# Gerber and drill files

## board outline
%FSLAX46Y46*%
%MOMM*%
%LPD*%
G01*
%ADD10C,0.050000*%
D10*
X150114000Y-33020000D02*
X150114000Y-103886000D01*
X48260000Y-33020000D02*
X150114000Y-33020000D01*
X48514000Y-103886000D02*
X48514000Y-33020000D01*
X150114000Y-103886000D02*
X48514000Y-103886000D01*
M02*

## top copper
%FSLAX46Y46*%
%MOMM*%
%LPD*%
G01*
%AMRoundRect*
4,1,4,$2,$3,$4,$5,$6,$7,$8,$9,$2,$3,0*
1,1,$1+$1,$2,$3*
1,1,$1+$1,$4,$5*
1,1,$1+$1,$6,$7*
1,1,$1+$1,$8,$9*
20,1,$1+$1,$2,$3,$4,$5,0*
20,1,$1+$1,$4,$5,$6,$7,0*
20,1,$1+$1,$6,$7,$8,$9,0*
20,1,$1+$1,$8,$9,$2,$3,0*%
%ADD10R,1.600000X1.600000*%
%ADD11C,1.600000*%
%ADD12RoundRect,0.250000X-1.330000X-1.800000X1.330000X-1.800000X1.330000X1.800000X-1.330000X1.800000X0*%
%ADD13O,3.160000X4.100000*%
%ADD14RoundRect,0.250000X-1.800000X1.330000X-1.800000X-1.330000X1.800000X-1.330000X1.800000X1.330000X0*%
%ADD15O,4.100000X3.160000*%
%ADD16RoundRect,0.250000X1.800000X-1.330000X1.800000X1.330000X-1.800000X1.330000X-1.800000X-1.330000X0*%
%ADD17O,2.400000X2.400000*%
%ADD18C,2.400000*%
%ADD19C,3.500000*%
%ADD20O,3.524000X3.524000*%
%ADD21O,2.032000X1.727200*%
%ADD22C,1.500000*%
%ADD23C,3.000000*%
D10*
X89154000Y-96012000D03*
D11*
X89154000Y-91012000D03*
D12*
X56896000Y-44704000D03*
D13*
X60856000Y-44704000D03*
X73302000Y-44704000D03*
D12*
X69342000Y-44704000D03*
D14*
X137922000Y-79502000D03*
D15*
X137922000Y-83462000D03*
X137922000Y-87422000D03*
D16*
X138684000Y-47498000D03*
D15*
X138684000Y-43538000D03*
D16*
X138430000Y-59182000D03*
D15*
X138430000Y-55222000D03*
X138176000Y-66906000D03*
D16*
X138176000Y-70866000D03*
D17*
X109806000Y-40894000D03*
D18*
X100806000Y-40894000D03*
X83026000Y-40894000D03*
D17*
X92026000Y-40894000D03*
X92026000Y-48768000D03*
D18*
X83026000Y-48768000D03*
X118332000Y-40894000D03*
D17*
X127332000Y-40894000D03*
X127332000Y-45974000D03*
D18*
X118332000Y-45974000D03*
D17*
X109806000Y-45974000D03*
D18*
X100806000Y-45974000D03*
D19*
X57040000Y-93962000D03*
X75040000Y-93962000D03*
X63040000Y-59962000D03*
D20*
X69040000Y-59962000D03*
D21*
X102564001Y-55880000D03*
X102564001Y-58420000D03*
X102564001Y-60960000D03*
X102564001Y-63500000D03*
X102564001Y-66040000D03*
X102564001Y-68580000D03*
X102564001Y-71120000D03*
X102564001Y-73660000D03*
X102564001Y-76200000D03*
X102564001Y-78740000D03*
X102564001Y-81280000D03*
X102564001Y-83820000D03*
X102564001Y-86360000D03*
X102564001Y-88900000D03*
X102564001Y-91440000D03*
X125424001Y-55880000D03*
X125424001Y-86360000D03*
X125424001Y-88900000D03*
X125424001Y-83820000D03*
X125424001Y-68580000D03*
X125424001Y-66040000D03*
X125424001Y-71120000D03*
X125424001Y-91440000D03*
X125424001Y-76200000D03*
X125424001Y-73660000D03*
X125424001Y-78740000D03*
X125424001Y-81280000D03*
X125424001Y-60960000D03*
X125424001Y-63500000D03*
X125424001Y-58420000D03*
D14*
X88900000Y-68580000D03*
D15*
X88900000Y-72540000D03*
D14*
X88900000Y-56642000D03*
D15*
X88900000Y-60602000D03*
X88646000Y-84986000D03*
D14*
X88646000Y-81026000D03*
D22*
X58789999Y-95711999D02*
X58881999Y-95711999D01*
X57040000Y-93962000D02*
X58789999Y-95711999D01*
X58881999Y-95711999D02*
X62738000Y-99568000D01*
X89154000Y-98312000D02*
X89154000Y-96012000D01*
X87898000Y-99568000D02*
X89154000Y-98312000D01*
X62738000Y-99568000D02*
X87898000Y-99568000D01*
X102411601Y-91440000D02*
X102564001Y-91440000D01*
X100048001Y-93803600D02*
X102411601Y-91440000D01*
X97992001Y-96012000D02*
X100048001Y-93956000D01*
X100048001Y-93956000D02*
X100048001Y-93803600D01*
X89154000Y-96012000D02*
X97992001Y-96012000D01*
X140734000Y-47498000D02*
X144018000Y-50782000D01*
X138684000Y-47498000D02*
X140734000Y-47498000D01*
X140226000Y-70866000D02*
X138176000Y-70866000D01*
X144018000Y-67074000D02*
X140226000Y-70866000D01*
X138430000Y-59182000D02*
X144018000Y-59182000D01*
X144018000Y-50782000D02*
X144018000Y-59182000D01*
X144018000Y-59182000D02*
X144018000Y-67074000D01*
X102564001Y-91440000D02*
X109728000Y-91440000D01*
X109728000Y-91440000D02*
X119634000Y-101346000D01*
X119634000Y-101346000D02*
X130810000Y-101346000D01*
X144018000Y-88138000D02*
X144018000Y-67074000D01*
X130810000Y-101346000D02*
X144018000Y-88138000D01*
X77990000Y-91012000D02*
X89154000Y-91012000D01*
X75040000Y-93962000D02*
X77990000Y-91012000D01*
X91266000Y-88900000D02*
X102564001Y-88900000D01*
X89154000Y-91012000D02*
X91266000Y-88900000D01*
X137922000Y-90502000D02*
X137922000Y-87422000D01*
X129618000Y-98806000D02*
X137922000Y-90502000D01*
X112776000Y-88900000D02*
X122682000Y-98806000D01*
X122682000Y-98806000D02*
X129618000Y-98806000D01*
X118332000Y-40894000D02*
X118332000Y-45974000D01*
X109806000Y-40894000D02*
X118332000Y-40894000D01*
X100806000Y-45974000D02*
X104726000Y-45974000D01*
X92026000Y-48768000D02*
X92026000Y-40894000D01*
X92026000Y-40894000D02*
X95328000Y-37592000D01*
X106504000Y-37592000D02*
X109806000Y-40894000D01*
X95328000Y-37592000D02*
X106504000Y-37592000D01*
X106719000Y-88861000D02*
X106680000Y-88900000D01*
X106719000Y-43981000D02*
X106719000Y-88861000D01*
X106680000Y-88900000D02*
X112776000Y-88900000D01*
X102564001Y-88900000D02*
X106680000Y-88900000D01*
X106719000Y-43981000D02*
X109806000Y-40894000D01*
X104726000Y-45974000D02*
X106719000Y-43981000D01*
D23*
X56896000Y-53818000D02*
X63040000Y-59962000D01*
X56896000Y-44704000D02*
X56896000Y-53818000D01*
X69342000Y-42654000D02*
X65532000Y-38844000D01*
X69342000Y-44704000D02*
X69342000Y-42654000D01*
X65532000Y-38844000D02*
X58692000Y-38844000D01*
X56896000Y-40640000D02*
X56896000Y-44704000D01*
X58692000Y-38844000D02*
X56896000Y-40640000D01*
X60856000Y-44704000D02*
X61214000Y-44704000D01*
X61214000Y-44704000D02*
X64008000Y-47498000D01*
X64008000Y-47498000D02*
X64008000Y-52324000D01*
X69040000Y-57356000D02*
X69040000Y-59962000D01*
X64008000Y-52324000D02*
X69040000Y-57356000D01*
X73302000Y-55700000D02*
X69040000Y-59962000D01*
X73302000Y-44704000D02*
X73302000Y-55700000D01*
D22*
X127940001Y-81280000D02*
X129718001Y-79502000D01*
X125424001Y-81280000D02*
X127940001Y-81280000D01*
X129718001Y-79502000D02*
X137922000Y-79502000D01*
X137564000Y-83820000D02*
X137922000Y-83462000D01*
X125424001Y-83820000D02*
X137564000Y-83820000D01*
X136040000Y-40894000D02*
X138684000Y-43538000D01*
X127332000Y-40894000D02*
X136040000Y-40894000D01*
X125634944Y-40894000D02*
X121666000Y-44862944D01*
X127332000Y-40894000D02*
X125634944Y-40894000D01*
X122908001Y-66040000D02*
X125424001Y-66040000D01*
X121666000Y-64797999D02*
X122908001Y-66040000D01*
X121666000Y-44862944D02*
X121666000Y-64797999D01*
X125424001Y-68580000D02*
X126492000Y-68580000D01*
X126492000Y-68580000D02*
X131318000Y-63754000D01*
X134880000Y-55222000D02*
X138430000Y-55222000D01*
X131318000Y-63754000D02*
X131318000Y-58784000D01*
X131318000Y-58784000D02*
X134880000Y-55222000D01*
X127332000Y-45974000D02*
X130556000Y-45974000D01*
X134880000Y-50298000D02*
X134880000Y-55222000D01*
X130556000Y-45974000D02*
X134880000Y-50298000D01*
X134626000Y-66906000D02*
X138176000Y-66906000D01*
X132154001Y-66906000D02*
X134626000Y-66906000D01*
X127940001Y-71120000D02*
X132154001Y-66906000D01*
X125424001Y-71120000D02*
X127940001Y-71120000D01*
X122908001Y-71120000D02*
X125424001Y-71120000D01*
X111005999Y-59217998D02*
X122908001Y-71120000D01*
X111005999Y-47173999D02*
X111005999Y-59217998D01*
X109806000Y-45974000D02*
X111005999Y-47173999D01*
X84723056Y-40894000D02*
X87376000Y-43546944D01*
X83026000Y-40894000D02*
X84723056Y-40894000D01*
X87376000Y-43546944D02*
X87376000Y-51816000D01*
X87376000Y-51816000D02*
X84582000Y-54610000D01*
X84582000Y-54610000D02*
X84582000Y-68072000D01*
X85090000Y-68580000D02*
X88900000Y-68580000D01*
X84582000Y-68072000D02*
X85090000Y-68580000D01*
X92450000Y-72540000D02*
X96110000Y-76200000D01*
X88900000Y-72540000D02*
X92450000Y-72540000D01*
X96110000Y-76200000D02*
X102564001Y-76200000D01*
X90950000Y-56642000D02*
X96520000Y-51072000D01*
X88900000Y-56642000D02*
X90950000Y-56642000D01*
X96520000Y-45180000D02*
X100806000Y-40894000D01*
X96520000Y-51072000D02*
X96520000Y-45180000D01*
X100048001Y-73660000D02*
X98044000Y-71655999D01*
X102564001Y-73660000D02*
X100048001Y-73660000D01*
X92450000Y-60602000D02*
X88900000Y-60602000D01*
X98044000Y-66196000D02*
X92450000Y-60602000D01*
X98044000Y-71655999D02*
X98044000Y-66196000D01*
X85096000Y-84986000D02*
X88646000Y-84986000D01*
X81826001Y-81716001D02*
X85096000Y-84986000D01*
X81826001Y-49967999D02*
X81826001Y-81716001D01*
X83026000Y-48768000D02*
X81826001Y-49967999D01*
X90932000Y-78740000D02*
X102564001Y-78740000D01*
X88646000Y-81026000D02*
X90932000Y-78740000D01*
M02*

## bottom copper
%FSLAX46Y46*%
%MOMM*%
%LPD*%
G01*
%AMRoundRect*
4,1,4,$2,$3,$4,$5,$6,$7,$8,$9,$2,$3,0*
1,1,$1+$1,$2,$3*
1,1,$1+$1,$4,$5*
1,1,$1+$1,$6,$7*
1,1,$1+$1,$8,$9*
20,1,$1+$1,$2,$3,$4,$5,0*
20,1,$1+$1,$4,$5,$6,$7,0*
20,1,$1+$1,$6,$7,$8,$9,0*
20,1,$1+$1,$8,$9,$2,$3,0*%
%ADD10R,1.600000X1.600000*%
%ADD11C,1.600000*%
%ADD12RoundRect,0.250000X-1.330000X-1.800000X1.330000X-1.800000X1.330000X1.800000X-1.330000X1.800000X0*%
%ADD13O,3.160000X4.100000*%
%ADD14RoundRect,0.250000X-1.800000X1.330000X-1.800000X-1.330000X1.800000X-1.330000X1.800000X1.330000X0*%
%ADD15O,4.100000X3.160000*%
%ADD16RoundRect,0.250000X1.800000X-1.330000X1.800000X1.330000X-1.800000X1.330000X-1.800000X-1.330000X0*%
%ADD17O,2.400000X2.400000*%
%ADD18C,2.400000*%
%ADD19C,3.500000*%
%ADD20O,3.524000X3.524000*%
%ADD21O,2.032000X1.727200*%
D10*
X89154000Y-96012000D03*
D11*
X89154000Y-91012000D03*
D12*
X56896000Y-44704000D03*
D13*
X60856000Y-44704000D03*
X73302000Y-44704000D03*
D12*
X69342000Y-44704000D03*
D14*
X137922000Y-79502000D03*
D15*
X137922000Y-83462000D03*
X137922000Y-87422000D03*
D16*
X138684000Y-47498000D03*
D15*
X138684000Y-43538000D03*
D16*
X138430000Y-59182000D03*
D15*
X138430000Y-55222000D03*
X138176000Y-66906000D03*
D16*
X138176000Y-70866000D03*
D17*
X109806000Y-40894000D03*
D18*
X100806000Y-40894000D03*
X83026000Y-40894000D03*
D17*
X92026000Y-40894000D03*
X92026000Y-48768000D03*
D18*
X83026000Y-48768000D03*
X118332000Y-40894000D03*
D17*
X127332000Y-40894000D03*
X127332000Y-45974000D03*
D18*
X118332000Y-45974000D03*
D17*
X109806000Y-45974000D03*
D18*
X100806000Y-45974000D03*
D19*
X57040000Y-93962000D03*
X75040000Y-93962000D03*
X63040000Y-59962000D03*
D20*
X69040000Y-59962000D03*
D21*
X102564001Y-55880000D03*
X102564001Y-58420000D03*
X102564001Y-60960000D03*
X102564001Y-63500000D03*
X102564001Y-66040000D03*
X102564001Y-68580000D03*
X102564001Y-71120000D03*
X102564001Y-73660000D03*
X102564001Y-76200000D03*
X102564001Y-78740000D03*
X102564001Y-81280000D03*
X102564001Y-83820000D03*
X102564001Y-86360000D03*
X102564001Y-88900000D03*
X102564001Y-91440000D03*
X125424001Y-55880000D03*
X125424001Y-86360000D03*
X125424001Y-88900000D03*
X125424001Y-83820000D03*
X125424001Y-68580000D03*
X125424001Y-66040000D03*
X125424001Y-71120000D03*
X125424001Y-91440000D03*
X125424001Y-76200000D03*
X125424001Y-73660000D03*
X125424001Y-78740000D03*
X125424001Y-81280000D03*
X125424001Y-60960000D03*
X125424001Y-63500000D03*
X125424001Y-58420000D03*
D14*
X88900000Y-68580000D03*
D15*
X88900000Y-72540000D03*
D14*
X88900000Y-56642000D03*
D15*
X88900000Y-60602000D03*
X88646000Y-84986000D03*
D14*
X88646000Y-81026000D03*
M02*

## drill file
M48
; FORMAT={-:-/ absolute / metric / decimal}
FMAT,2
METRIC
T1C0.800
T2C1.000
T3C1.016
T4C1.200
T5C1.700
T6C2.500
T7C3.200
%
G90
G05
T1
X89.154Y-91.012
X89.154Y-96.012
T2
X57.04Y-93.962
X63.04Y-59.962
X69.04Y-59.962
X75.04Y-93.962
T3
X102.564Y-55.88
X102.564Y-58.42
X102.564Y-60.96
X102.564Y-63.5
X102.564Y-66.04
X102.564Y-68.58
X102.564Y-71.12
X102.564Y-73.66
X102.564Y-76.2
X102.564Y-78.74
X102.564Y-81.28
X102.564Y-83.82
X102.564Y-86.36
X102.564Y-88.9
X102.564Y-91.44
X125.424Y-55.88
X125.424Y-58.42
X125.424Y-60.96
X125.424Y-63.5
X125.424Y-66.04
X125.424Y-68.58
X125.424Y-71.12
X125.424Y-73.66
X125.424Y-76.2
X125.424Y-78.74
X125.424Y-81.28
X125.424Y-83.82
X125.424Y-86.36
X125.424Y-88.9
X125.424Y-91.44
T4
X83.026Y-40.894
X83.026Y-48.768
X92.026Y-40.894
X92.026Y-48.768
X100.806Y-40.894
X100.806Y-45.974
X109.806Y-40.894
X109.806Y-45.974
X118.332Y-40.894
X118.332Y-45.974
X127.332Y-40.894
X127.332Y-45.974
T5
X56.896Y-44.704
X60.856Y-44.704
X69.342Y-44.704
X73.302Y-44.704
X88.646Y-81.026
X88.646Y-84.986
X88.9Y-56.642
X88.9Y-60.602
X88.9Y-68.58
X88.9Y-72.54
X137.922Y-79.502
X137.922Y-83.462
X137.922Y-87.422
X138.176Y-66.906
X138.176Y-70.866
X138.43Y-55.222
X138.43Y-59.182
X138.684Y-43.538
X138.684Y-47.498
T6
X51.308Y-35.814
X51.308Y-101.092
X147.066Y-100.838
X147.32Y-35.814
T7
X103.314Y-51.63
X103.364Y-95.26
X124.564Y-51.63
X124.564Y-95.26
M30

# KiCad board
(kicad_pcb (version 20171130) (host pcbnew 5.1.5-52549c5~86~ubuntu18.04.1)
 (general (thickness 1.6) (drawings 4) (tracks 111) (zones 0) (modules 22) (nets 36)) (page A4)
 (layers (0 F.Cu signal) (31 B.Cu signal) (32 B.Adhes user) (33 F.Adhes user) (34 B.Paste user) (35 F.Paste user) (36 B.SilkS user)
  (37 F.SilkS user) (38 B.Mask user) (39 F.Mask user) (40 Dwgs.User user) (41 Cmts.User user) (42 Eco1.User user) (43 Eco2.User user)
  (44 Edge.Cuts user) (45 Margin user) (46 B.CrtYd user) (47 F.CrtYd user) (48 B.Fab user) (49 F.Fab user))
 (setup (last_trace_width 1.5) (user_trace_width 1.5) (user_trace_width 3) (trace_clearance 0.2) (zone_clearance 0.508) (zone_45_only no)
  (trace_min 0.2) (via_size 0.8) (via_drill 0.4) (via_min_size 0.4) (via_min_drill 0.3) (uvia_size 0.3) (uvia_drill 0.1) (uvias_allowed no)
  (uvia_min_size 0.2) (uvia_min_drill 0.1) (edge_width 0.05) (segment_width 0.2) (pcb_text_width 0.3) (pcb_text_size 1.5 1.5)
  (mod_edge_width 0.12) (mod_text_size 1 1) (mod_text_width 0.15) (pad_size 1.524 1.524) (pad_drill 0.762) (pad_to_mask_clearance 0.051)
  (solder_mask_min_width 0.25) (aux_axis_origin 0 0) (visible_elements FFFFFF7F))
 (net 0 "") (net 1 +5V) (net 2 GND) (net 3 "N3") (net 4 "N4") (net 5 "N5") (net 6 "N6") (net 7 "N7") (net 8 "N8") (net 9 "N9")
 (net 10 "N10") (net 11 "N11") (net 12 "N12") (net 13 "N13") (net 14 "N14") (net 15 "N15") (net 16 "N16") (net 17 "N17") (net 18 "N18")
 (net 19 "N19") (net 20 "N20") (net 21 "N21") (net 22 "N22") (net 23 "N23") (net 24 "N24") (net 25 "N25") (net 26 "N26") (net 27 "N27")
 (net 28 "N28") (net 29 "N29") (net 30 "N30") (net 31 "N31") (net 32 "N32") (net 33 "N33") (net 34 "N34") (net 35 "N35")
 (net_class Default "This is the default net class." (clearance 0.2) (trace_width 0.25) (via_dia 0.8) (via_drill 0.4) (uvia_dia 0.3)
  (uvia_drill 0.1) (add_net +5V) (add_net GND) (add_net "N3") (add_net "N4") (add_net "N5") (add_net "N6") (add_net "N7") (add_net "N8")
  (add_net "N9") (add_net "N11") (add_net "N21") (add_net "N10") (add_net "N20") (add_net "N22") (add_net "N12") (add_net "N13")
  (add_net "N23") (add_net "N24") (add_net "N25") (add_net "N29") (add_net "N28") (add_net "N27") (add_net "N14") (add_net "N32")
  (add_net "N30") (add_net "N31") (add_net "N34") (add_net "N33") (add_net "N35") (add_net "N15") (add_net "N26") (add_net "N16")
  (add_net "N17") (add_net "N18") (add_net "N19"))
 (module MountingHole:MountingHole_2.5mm (layer F.Cu) (at 51.308 35.814)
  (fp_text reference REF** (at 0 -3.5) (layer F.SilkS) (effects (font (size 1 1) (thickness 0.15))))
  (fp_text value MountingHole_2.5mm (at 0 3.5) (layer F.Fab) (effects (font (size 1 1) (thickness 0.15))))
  (pad 1 np_thru_hole circle (at 0 0) (size 2.5 2.5) (drill 2.5) (layers *.Cu *.Mask)))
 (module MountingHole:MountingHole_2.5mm (layer F.Cu) (at 51.308 101.092)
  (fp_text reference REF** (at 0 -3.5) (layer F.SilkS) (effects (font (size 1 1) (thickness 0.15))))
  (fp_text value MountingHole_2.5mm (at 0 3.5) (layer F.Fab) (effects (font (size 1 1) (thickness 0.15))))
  (pad 1 np_thru_hole circle (at 0 0) (size 2.5 2.5) (drill 2.5) (layers *.Cu *.Mask)))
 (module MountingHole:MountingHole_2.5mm (layer F.Cu) (at 147.066 100.838)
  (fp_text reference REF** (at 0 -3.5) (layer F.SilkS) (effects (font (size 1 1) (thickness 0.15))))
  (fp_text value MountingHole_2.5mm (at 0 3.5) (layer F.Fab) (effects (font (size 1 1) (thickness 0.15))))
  (pad 1 np_thru_hole circle (at 0 0) (size 2.5 2.5) (drill 2.5) (layers *.Cu *.Mask)))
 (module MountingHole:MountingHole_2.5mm (layer F.Cu) (at 147.32 35.814)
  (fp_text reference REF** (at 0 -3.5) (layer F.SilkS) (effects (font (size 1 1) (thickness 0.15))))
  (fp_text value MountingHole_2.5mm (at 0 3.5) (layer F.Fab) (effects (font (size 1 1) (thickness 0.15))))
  (pad 1 np_thru_hole circle (at 0 0) (size 2.5 2.5) (drill 2.5) (layers *.Cu *.Mask)))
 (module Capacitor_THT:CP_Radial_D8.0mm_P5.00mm (layer F.Cu) (at 89.154 96.012 90)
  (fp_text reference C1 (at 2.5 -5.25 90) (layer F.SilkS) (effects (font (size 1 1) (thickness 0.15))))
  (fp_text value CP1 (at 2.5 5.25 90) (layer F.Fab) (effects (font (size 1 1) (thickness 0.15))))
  (pad 1 thru_hole rect (at 0 0 90) (size 1.6 1.6) (drill 0.8) (layers *.Cu *.Mask) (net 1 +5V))
  (pad 2 thru_hole circle (at 5 0 90) (size 1.6 1.6) (drill 0.8) (layers *.Cu *.Mask) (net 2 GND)))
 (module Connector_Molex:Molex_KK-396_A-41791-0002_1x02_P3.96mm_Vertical (layer F.Cu) (at 56.896 44.704)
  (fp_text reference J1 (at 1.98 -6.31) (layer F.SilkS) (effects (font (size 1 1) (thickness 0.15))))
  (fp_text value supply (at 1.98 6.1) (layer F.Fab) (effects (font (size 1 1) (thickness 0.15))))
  (pad 1 thru_hole roundrect (at 0 0) (size 3.16 4.1) (drill 1.7) (layers *.Cu *.Mask) (roundrect_rratio 0.079114) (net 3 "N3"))
  (pad 2 thru_hole oval (at 3.96 0) (size 3.16 4.1) (drill 1.7) (layers *.Cu *.Mask) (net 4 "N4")))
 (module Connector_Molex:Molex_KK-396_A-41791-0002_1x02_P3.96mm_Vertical (layer F.Cu) (at 69.342 44.704)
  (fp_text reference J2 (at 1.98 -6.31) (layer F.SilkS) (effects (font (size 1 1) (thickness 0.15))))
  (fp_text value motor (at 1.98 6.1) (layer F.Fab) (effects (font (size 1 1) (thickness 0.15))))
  (pad 2 thru_hole oval (at 3.96 0) (size 3.16 4.1) (drill 1.7) (layers *.Cu *.Mask) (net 4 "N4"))
  (pad 1 thru_hole roundrect (at 0 0) (size 3.16 4.1) (drill 1.7) (layers *.Cu *.Mask) (roundrect_rratio 0.079114) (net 3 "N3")))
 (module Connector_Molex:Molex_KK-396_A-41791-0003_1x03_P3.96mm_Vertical (layer F.Cu) (at 137.922 79.502 270)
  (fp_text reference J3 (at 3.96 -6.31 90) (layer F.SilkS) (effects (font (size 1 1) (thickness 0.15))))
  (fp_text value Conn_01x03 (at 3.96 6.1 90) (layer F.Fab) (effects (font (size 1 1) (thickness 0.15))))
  (pad 1 thru_hole roundrect (at 0 0 270) (size 3.16 4.1) (drill 1.7) (layers *.Cu *.Mask) (roundrect_rratio 0.079114) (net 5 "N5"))
  (pad 2 thru_hole oval (at 3.96 0 270) (size 3.16 4.1) (drill 1.7) (layers *.Cu *.Mask) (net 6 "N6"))
  (pad 3 thru_hole oval (at 7.92 0 270) (size 3.16 4.1) (drill 1.7) (layers *.Cu *.Mask) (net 2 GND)))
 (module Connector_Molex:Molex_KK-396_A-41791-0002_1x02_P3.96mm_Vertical (layer F.Cu) (at 138.684 47.498 90)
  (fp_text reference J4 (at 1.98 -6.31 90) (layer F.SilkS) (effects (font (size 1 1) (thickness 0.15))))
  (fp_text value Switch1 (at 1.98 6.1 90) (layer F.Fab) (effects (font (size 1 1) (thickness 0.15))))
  (pad 1 thru_hole roundrect (at 0 0 90) (size 3.16 4.1) (drill 1.7) (layers *.Cu *.Mask) (roundrect_rratio 0.079114) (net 1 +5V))
  (pad 2 thru_hole oval (at 3.96 0 90) (size 3.16 4.1) (drill 1.7) (layers *.Cu *.Mask) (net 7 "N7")))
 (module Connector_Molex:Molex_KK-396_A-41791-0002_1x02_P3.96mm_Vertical (layer F.Cu) (at 138.43 59.182 90)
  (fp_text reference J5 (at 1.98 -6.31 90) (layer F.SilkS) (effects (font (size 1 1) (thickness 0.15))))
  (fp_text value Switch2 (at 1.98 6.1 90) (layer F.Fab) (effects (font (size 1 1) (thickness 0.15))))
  (pad 1 thru_hole roundrect (at 0 0 90) (size 3.16 4.1) (drill 1.7) (layers *.Cu *.Mask) (roundrect_rratio 0.079114) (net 1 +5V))
  (pad 2 thru_hole oval (at 3.96 0 90) (size 3.16 4.1) (drill 1.7) (layers *.Cu *.Mask) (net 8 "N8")))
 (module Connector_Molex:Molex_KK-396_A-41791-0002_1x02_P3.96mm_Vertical (layer F.Cu) (at 138.176 70.866 90)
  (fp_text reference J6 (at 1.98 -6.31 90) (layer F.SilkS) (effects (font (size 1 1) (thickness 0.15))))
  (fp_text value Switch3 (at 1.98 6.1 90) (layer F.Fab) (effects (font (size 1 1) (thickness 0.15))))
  (pad 2 thru_hole oval (at 3.96 0 90) (size 3.16 4.1) (drill 1.7) (layers *.Cu *.Mask) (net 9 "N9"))
  (pad 1 thru_hole roundrect (at 0 0 90) (size 3.16 4.1) (drill 1.7) (layers *.Cu *.Mask) (roundrect_rratio 0.079114) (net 1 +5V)))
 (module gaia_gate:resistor (layer F.Cu) (at 98.806 40.894)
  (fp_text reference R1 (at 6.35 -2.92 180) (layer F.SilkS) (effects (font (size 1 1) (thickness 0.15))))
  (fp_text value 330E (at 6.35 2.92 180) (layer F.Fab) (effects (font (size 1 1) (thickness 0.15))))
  (pad 2 thru_hole oval (at 11 0) (size 2.4 2.4) (drill 1.2) (layers *.Cu *.Mask) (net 2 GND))
  (pad 1 thru_hole circle (at 2 0) (size 2.4 2.4) (drill 1.2) (layers *.Cu *.Mask) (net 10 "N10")))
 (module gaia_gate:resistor (layer F.Cu) (at 81.026 40.894)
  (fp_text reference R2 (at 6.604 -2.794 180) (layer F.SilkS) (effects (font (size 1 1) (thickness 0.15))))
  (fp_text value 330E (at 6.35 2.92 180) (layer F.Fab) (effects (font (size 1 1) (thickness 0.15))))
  (pad 1 thru_hole circle (at 2 0) (size 2.4 2.4) (drill 1.2) (layers *.Cu *.Mask) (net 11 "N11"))
  (pad 2 thru_hole oval (at 11 0) (size 2.4 2.4) (drill 1.2) (layers *.Cu *.Mask) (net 2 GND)))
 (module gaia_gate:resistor (layer F.Cu) (at 81.026 48.768)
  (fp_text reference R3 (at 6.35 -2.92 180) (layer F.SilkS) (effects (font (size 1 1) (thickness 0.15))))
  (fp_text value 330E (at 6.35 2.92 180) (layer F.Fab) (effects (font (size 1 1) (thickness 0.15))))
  (pad 2 thru_hole oval (at 11 0) (size 2.4 2.4) (drill 1.2) (layers *.Cu *.Mask) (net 2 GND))
  (pad 1 thru_hole circle (at 2 0) (size 2.4 2.4) (drill 1.2) (layers *.Cu *.Mask) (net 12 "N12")))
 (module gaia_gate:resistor (layer F.Cu) (at 116.332 40.894)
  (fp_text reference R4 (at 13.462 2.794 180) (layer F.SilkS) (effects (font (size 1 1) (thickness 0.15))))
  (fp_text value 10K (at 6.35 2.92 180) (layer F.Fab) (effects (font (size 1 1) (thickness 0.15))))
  (pad 1 thru_hole circle (at 2 0) (size 2.4 2.4) (drill 1.2) (layers *.Cu *.Mask) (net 2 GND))
  (pad 2 thru_hole oval (at 11 0) (size 2.4 2.4) (drill 1.2) (layers *.Cu *.Mask) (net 7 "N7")))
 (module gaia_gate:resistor (layer F.Cu) (at 116.332 45.974)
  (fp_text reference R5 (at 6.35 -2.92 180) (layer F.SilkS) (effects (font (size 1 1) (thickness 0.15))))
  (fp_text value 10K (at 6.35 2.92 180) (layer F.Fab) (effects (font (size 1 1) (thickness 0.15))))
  (pad 2 thru_hole oval (at 11 0) (size 2.4 2.4) (drill 1.2) (layers *.Cu *.Mask) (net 8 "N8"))
  (pad 1 thru_hole circle (at 2 0) (size 2.4 2.4) (drill 1.2) (layers *.Cu *.Mask) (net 2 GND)))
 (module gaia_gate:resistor (layer F.Cu) (at 98.806 45.974)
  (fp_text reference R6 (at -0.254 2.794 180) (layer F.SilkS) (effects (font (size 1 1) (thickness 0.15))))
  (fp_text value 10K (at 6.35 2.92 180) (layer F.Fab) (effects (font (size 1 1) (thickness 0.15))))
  (pad 2 thru_hole oval (at 11 0) (size 2.4 2.4) (drill 1.2) (layers *.Cu *.Mask) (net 9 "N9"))
  (pad 1 thru_hole circle (at 2 0) (size 2.4 2.4) (drill 1.2) (layers *.Cu *.Mask) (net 2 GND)))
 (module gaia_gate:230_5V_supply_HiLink (layer F.Cu) (at 66.04 76.962 270)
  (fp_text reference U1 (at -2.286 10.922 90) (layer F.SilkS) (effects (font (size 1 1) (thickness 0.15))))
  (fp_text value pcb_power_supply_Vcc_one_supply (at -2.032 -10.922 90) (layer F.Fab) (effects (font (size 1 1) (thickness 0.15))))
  (pad 3 thru_hole circle (at 17 9 270) (size 3.5 3.5) (drill 1) (layers *.Cu *.Mask) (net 1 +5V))
  (pad 4 thru_hole circle (at 17 -9 270) (size 3.5 3.5) (drill 1) (layers *.Cu *.Mask) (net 2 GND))
  (pad 2 thru_hole circle (at -17 3 270) (size 3.5 3.5) (drill 1) (layers *.Cu *.Mask) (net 3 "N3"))
  (pad 1 thru_hole oval (at -17 -3 270) (size 3.524 3.524) (drill 1) (layers *.Cu *.Mask) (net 4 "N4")))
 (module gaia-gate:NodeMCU (layer F.Cu) (at 102.564001 55.88)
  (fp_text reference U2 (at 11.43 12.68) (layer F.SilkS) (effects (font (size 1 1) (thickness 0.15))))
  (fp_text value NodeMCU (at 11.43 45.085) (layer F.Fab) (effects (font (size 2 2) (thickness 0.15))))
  (pad 1 thru_hole oval (at 0 0) (size 2.032 1.7272) (drill 1.016) (layers *.Cu *.Mask F.SilkS) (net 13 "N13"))
  (pad 2 thru_hole oval (at 0 2.54) (size 2.032 1.7272) (drill 1.016) (layers *.Cu *.Mask F.SilkS) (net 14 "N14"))
  (pad 3 thru_hole oval (at 0 5.08) (size 2.032 1.7272) (drill 1.016) (layers *.Cu *.Mask F.SilkS) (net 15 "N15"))
  (pad 4 thru_hole oval (at 0 7.62) (size 2.032 1.7272) (drill 1.016) (layers *.Cu *.Mask F.SilkS) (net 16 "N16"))
  (pad 5 thru_hole oval (at 0 10.16) (size 2.032 1.7272) (drill 1.016) (layers *.Cu *.Mask F.SilkS) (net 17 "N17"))
  (pad 6 thru_hole oval (at 0 12.7) (size 2.032 1.7272) (drill 1.016) (layers *.Cu *.Mask F.SilkS) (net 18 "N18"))
  (pad 7 thru_hole oval (at 0 15.24) (size 2.032 1.7272) (drill 1.016) (layers *.Cu *.Mask F.SilkS) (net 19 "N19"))
  (pad 8 thru_hole oval (at 0 17.78) (size 2.032 1.7272) (drill 1.016) (layers *.Cu *.Mask F.SilkS) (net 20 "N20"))
  (pad 9 thru_hole oval (at 0 20.32) (size 2.032 1.7272) (drill 1.016) (layers *.Cu *.Mask F.SilkS) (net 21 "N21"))
  (pad 10 thru_hole oval (at 0 22.86) (size 2.032 1.7272) (drill 1.016) (layers *.Cu *.Mask F.SilkS) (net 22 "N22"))
  (pad 11 thru_hole oval (at 0 25.4) (size 2.032 1.7272) (drill 1.016) (layers *.Cu *.Mask F.SilkS) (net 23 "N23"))
  (pad 12 thru_hole oval (at 0 27.94) (size 2.032 1.7272) (drill 1.016) (layers *.Cu *.Mask F.SilkS) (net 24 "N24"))
  (pad 13 thru_hole oval (at 0 30.48) (size 2.032 1.7272) (drill 1.016) (layers *.Cu *.Mask F.SilkS) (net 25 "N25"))
  (pad 14 thru_hole oval (at 0 33.02) (size 2.032 1.7272) (drill 1.016) (layers *.Cu *.Mask F.SilkS) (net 2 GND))
  (pad 15 thru_hole oval (at 0 35.56) (size 2.032 1.7272) (drill 1.016) (layers *.Cu *.Mask F.SilkS) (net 1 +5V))
  (pad 30 thru_hole oval (at 22.86 0) (size 2.032 1.7272) (drill 1.016) (layers *.Cu *.Mask F.SilkS) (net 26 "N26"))
  (pad 18 thru_hole oval (at 22.86 30.48) (size 2.032 1.7272) (drill 1.016) (layers *.Cu *.Mask F.SilkS) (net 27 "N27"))
  (pad 17 thru_hole oval (at 22.86 33.02) (size 2.032 1.7272) (drill 1.016) (layers *.Cu *.Mask F.SilkS) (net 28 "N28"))
  (pad 19 thru_hole oval (at 22.86 27.94) (size 2.032 1.7272) (drill 1.016) (layers *.Cu *.Mask F.SilkS) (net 6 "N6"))
  (pad 25 thru_hole oval (at 22.86 12.7) (size 2.032 1.7272) (drill 1.016) (layers *.Cu *.Mask F.SilkS) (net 8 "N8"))
  (pad 26 thru_hole oval (at 22.86 10.16) (size 2.032 1.7272) (drill 1.016) (layers *.Cu *.Mask F.SilkS) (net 7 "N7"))
  (pad 24 thru_hole oval (at 22.86 15.24) (size 2.032 1.7272) (drill 1.016) (layers *.Cu *.Mask F.SilkS) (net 9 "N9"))
  (pad 16 thru_hole oval (at 22.86 35.56) (size 2.032 1.7272) (drill 1.016) (layers *.Cu *.Mask F.SilkS) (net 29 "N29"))
  (pad 22 thru_hole oval (at 22.86 20.32) (size 2.032 1.7272) (drill 1.016) (layers *.Cu *.Mask F.SilkS) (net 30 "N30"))
  (pad 23 thru_hole oval (at 22.86 17.78) (size 2.032 1.7272) (drill 1.016) (layers *.Cu *.Mask F.SilkS) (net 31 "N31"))
  (pad 21 thru_hole oval (at 22.86 22.86) (size 2.032 1.7272) (drill 1.016) (layers *.Cu *.Mask F.SilkS) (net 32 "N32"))
  (pad 20 thru_hole oval (at 22.86 25.4) (size 2.032 1.7272) (drill 1.016) (layers *.Cu *.Mask F.SilkS) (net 5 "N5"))
  (pad 28 thru_hole oval (at 22.86 5.08) (size 2.032 1.7272) (drill 1.016) (layers *.Cu *.Mask F.SilkS) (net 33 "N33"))
  (pad 27 thru_hole oval (at 22.86 7.62) (size 2.032 1.7272) (drill 1.016) (layers *.Cu *.Mask F.SilkS) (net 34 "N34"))
  (pad 29 thru_hole oval (at 22.86 2.54) (size 2.032 1.7272) (drill 1.016) (layers *.Cu *.Mask F.SilkS) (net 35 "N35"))
  (pad "" np_thru_hole circle (at 0.8 39.38) (size 3.2 3.2) (drill 3.2) (layers *.Cu *.Mask))
  (pad "" np_thru_hole circle (at 22 39.38) (size 3.2 3.2) (drill 3.2) (layers *.Cu *.Mask))
  (pad "" np_thru_hole circle (at 22 -4.25) (size 3.2 3.2) (drill 3.2) (layers *.Cu *.Mask))
  (pad "" np_thru_hole circle (at 0.75 -4.25) (size 3.2 3.2) (drill 3.2) (layers *.Cu *.Mask)))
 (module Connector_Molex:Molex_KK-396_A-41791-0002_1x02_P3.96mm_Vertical (layer F.Cu) (at 88.9 68.58 270)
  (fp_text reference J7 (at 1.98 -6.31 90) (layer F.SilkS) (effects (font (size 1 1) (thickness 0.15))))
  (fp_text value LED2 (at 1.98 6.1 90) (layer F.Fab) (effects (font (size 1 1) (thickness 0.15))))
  (pad 1 thru_hole roundrect (at 0 0 270) (size 3.16 4.1) (drill 1.7) (layers *.Cu *.Mask) (roundrect_rratio 0.079114) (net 11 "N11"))
  (pad 2 thru_hole oval (at 3.96 0 270) (size 3.16 4.1) (drill 1.7) (layers *.Cu *.Mask) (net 21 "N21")))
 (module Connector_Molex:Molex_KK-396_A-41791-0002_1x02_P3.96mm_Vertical (layer F.Cu) (at 88.9 56.642 270)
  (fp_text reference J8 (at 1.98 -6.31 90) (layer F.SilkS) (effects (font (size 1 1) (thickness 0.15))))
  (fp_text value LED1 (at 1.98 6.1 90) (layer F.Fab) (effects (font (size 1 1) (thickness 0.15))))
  (pad 1 thru_hole roundrect (at 0 0 270) (size 3.16 4.1) (drill 1.7) (layers *.Cu *.Mask) (roundrect_rratio 0.079114) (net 10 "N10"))
  (pad 2 thru_hole oval (at 3.96 0 270) (size 3.16 4.1) (drill 1.7) (layers *.Cu *.Mask) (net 20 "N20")))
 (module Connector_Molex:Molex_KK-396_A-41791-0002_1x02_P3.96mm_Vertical (layer F.Cu) (at 88.646 81.026 270)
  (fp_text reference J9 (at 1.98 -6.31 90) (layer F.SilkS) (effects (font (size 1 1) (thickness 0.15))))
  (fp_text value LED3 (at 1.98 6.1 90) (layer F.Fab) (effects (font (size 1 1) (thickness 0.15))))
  (pad 2 thru_hole oval (at 3.96 0 270) (size 3.16 4.1) (drill 1.7) (layers *.Cu *.Mask) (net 12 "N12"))
  (pad 1 thru_hole roundrect (at 0 0 270) (size 3.16 4.1) (drill 1.7) (layers *.Cu *.Mask) (roundrect_rratio 0.079114) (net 22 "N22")))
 (gr_line (start 150.114 33.02) (end 150.114 103.886) (layer Edge.Cuts) (width 0.05))
 (gr_line (start 48.26 33.02) (end 150.114 33.02) (layer Edge.Cuts) (width 0.05))
 (gr_line (start 48.514 103.886) (end 48.514 33.02) (layer Edge.Cuts) (width 0.05))
 (gr_line (start 150.114 103.886) (end 48.514 103.886) (layer Edge.Cuts) (width 0.05))
 (segment (start 58.789999 95.711999) (end 58.881999 95.711999) (width 1.5) (layer F.Cu) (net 1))
 (segment (start 57.04 93.962) (end 58.789999 95.711999) (width 1.5) (layer F.Cu) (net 1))
 (segment (start 58.881999 95.711999) (end 62.738 99.568) (width 1.5) (layer F.Cu) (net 1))
 (segment (start 89.154 98.312) (end 89.154 96.012) (width 1.5) (layer F.Cu) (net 1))
 (segment (start 87.898 99.568) (end 89.154 98.312) (width 1.5) (layer F.Cu) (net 1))
 (segment (start 62.738 99.568) (end 87.898 99.568) (width 1.5) (layer F.Cu) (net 1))
 (segment (start 102.411601 91.44) (end 102.564001 91.44) (width 1.5) (layer F.Cu) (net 1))
 (segment (start 100.048001 93.8036) (end 102.411601 91.44) (width 1.5) (layer F.Cu) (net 1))
 (segment (start 97.992001 96.012) (end 100.048001 93.956) (width 1.5) (layer F.Cu) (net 1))
 (segment (start 100.048001 93.956) (end 100.048001 93.8036) (width 1.5) (layer F.Cu) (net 1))
 (segment (start 89.154 96.012) (end 97.992001 96.012) (width 1.5) (layer F.Cu) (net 1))
 (segment (start 140.734 47.498) (end 144.018 50.782) (width 1.5) (layer F.Cu) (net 1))
 (segment (start 138.684 47.498) (end 140.734 47.498) (width 1.5) (layer F.Cu) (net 1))
 (segment (start 140.226 70.866) (end 138.176 70.866) (width 1.5) (layer F.Cu) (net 1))
 (segment (start 144.018 67.074) (end 140.226 70.866) (width 1.5) (layer F.Cu) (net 1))
 (segment (start 138.43 59.182) (end 144.018 59.182) (width 1.5) (layer F.Cu) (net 1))
 (segment (start 144.018 50.782) (end 144.018 59.182) (width 1.5) (layer F.Cu) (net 1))
 (segment (start 144.018 59.182) (end 144.018 67.074) (width 1.5) (layer F.Cu) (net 1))
 (segment (start 102.564001 91.44) (end 109.728 91.44) (width 1.5) (layer F.Cu) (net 1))
 (segment (start 109.728 91.44) (end 119.634 101.346) (width 1.5) (layer F.Cu) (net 1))
 (segment (start 119.634 101.346) (end 130.81 101.346) (width 1.5) (layer F.Cu) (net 1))
 (segment (start 144.018 88.138) (end 144.018 67.074) (width 1.5) (layer F.Cu) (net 1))
 (segment (start 130.81 101.346) (end 144.018 88.138) (width 1.5) (layer F.Cu) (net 1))
 (segment (start 77.99 91.012) (end 89.154 91.012) (width 1.5) (layer F.Cu) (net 2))
 (segment (start 75.04 93.962) (end 77.99 91.012) (width 1.5) (layer F.Cu) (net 2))
 (segment (start 91.266 88.9) (end 102.564001 88.9) (width 1.5) (layer F.Cu) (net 2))
 (segment (start 89.154 91.012) (end 91.266 88.9) (width 1.5) (layer F.Cu) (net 2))
 (segment (start 137.922 90.502) (end 137.922 87.422) (width 1.5) (layer F.Cu) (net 2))
 (segment (start 129.618 98.806) (end 137.922 90.502) (width 1.5) (layer F.Cu) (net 2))
 (segment (start 112.776 88.9) (end 122.682 98.806) (width 1.5) (layer F.Cu) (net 2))
 (segment (start 122.682 98.806) (end 129.618 98.806) (width 1.5) (layer F.Cu) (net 2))
 (segment (start 118.332 40.894) (end 118.332 45.974) (width 1.5) (layer F.Cu) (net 2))
 (segment (start 109.806 40.894) (end 118.332 40.894) (width 1.5) (layer F.Cu) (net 2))
 (segment (start 100.806 45.974) (end 104.726 45.974) (width 1.5) (layer F.Cu) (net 2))
 (segment (start 92.026 48.768) (end 92.026 40.894) (width 1.5) (layer F.Cu) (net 2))
 (segment (start 92.026 40.894) (end 95.328 37.592) (width 1.5) (layer F.Cu) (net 2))
 (segment (start 106.504 37.592) (end 109.806 40.894) (width 1.5) (layer F.Cu) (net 2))
 (segment (start 95.328 37.592) (end 106.504 37.592) (width 1.5) (layer F.Cu) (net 2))
 (segment (start 106.719 88.861) (end 106.68 88.9) (width 1.5) (layer F.Cu) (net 2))
 (segment (start 106.719 43.981) (end 106.719 88.861) (width 1.5) (layer F.Cu) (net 2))
 (segment (start 106.68 88.9) (end 112.776 88.9) (width 1.5) (layer F.Cu) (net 2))
 (segment (start 102.564001 88.9) (end 106.68 88.9) (width 1.5) (layer F.Cu) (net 2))
 (segment (start 106.719 43.981) (end 109.806 40.894) (width 1.5) (layer F.Cu) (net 2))
 (segment (start 104.726 45.974) (end 106.719 43.981) (width 1.5) (layer F.Cu) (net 2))
 (segment (start 56.896 53.818) (end 63.04 59.962) (width 3) (layer F.Cu) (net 3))
 (segment (start 56.896 44.704) (end 56.896 53.818) (width 3) (layer F.Cu) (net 3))
 (segment (start 69.342 42.654) (end 65.532 38.844) (width 3) (layer F.Cu) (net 3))
 (segment (start 69.342 44.704) (end 69.342 42.654) (width 3) (layer F.Cu) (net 3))
 (segment (start 65.532 38.844) (end 58.692 38.844) (width 3) (layer F.Cu) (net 3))
 (segment (start 56.896 40.64) (end 56.896 44.704) (width 3) (layer F.Cu) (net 3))
 (segment (start 58.692 38.844) (end 56.896 40.64) (width 3) (layer F.Cu) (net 3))
 (segment (start 60.856 44.704) (end 61.214 44.704) (width 3) (layer F.Cu) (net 4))
 (segment (start 61.214 44.704) (end 64.008 47.498) (width 3) (layer F.Cu) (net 4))
 (segment (start 64.008 47.498) (end 64.008 52.324) (width 3) (layer F.Cu) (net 4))
 (segment (start 69.04 57.356) (end 69.04 59.962) (width 3) (layer F.Cu) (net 4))
 (segment (start 64.008 52.324) (end 69.04 57.356) (width 3) (layer F.Cu) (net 4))
 (segment (start 73.302 55.7) (end 69.04 59.962) (width 3) (layer F.Cu) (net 4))
 (segment (start 73.302 44.704) (end 73.302 55.7) (width 3) (layer F.Cu) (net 4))
 (segment (start 127.940001 81.28) (end 129.718001 79.502) (width 1.5) (layer F.Cu) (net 5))
 (segment (start 125.424001 81.28) (end 127.940001 81.28) (width 1.5) (layer F.Cu) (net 5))
 (segment (start 129.718001 79.502) (end 137.922 79.502) (width 1.5) (layer F.Cu) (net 5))
 (segment (start 137.564 83.82) (end 137.922 83.462) (width 1.5) (layer F.Cu) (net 6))
 (segment (start 125.424001 83.82) (end 137.564 83.82) (width 1.5) (layer F.Cu) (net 6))
 (segment (start 136.04 40.894) (end 138.684 43.538) (width 1.5) (layer F.Cu) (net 7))
 (segment (start 127.332 40.894) (end 136.04 40.894) (width 1.5) (layer F.Cu) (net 7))
 (segment (start 125.634944 40.894) (end 121.666 44.862944) (width 1.5) (layer F.Cu) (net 7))
 (segment (start 127.332 40.894) (end 125.634944 40.894) (width 1.5) (layer F.Cu) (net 7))
 (segment (start 122.908001 66.04) (end 125.424001 66.04) (width 1.5) (layer F.Cu) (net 7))
 (segment (start 121.666 64.797999) (end 122.908001 66.04) (width 1.5) (layer F.Cu) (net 7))
 (segment (start 121.666 44.862944) (end 121.666 64.797999) (width 1.5) (layer F.Cu) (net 7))
 (segment (start 125.424001 68.58) (end 126.492 68.58) (width 1.5) (layer F.Cu) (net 8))
 (segment (start 126.492 68.58) (end 131.318 63.754) (width 1.5) (layer F.Cu) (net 8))
 (segment (start 134.88 55.222) (end 138.43 55.222) (width 1.5) (layer F.Cu) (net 8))
 (segment (start 131.318 63.754) (end 131.318 58.784) (width 1.5) (layer F.Cu) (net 8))
 (segment (start 131.318 58.784) (end 134.88 55.222) (width 1.5) (layer F.Cu) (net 8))
 (segment (start 127.332 45.974) (end 130.556 45.974) (width 1.5) (layer F.Cu) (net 8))
 (segment (start 134.88 50.298) (end 134.88 55.222) (width 1.5) (layer F.Cu) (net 8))
 (segment (start 130.556 45.974) (end 134.88 50.298) (width 1.5) (layer F.Cu) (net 8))
 (segment (start 134.626 66.906) (end 138.176 66.906) (width 1.5) (layer F.Cu) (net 9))
 (segment (start 132.154001 66.906) (end 134.626 66.906) (width 1.5) (layer F.Cu) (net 9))
 (segment (start 127.940001 71.12) (end 132.154001 66.906) (width 1.5) (layer F.Cu) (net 9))
 (segment (start 125.424001 71.12) (end 127.940001 71.12) (width 1.5) (layer F.Cu) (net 9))
 (segment (start 122.908001 71.12) (end 125.424001 71.12) (width 1.5) (layer F.Cu) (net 9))
 (segment (start 111.005999 59.217998) (end 122.908001 71.12) (width 1.5) (layer F.Cu) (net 9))
 (segment (start 111.005999 47.173999) (end 111.005999 59.217998) (width 1.5) (layer F.Cu) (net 9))
 (segment (start 109.806 45.974) (end 111.005999 47.173999) (width 1.5) (layer F.Cu) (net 9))
 (segment (start 84.723056 40.894) (end 87.376 43.546944) (width 1.5) (layer F.Cu) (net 11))
 (segment (start 83.026 40.894) (end 84.723056 40.894) (width 1.5) (layer F.Cu) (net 11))
 (segment (start 87.376 43.546944) (end 87.376 51.816) (width 1.5) (layer F.Cu) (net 11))
 (segment (start 87.376 51.816) (end 84.582 54.61) (width 1.5) (layer F.Cu) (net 11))
 (segment (start 84.582 54.61) (end 84.582 68.072) (width 1.5) (layer F.Cu) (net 11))
 (segment (start 85.09 68.58) (end 88.9 68.58) (width 1.5) (layer F.Cu) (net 11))
 (segment (start 84.582 68.072) (end 85.09 68.58) (width 1.5) (layer F.Cu) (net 11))
 (segment (start 92.45 72.54) (end 96.11 76.2) (width 1.5) (layer F.Cu) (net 21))
 (segment (start 88.9 72.54) (end 92.45 72.54) (width 1.5) (layer F.Cu) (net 21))
 (segment (start 96.11 76.2) (end 102.564001 76.2) (width 1.5) (layer F.Cu) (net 21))
 (segment (start 90.95 56.642) (end 96.52 51.072) (width 1.5) (layer F.Cu) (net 10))
 (segment (start 88.9 56.642) (end 90.95 56.642) (width 1.5) (layer F.Cu) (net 10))
 (segment (start 96.52 45.18) (end 100.806 40.894) (width 1.5) (layer F.Cu) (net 10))
 (segment (start 96.52 51.072) (end 96.52 45.18) (width 1.5) (layer F.Cu) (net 10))
 (segment (start 100.048001 73.66) (end 98.044 71.655999) (width 1.5) (layer F.Cu) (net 20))
 (segment (start 102.564001 73.66) (end 100.048001 73.66) (width 1.5) (layer F.Cu) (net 20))
 (segment (start 92.45 60.602) (end 88.9 60.602) (width 1.5) (layer F.Cu) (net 20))
 (segment (start 98.044 66.196) (end 92.45 60.602) (width 1.5) (layer F.Cu) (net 20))
 (segment (start 98.044 71.655999) (end 98.044 66.196) (width 1.5) (layer F.Cu) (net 20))
 (segment (start 85.096 84.986) (end 88.646 84.986) (width 1.5) (layer F.Cu) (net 12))
 (segment (start 81.826001 81.716001) (end 85.096 84.986) (width 1.5) (layer F.Cu) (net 12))
 (segment (start 81.826001 49.967999) (end 81.826001 81.716001) (width 1.5) (layer F.Cu) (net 12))
 (segment (start 83.026 48.768) (end 81.826001 49.967999) (width 1.5) (layer F.Cu) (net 12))
 (segment (start 90.932 78.74) (end 102.564001 78.74) (width 1.5) (layer F.Cu) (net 22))
 (segment (start 88.646 81.026) (end 90.932 78.74) (width 1.5) (layer F.Cu) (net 22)))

